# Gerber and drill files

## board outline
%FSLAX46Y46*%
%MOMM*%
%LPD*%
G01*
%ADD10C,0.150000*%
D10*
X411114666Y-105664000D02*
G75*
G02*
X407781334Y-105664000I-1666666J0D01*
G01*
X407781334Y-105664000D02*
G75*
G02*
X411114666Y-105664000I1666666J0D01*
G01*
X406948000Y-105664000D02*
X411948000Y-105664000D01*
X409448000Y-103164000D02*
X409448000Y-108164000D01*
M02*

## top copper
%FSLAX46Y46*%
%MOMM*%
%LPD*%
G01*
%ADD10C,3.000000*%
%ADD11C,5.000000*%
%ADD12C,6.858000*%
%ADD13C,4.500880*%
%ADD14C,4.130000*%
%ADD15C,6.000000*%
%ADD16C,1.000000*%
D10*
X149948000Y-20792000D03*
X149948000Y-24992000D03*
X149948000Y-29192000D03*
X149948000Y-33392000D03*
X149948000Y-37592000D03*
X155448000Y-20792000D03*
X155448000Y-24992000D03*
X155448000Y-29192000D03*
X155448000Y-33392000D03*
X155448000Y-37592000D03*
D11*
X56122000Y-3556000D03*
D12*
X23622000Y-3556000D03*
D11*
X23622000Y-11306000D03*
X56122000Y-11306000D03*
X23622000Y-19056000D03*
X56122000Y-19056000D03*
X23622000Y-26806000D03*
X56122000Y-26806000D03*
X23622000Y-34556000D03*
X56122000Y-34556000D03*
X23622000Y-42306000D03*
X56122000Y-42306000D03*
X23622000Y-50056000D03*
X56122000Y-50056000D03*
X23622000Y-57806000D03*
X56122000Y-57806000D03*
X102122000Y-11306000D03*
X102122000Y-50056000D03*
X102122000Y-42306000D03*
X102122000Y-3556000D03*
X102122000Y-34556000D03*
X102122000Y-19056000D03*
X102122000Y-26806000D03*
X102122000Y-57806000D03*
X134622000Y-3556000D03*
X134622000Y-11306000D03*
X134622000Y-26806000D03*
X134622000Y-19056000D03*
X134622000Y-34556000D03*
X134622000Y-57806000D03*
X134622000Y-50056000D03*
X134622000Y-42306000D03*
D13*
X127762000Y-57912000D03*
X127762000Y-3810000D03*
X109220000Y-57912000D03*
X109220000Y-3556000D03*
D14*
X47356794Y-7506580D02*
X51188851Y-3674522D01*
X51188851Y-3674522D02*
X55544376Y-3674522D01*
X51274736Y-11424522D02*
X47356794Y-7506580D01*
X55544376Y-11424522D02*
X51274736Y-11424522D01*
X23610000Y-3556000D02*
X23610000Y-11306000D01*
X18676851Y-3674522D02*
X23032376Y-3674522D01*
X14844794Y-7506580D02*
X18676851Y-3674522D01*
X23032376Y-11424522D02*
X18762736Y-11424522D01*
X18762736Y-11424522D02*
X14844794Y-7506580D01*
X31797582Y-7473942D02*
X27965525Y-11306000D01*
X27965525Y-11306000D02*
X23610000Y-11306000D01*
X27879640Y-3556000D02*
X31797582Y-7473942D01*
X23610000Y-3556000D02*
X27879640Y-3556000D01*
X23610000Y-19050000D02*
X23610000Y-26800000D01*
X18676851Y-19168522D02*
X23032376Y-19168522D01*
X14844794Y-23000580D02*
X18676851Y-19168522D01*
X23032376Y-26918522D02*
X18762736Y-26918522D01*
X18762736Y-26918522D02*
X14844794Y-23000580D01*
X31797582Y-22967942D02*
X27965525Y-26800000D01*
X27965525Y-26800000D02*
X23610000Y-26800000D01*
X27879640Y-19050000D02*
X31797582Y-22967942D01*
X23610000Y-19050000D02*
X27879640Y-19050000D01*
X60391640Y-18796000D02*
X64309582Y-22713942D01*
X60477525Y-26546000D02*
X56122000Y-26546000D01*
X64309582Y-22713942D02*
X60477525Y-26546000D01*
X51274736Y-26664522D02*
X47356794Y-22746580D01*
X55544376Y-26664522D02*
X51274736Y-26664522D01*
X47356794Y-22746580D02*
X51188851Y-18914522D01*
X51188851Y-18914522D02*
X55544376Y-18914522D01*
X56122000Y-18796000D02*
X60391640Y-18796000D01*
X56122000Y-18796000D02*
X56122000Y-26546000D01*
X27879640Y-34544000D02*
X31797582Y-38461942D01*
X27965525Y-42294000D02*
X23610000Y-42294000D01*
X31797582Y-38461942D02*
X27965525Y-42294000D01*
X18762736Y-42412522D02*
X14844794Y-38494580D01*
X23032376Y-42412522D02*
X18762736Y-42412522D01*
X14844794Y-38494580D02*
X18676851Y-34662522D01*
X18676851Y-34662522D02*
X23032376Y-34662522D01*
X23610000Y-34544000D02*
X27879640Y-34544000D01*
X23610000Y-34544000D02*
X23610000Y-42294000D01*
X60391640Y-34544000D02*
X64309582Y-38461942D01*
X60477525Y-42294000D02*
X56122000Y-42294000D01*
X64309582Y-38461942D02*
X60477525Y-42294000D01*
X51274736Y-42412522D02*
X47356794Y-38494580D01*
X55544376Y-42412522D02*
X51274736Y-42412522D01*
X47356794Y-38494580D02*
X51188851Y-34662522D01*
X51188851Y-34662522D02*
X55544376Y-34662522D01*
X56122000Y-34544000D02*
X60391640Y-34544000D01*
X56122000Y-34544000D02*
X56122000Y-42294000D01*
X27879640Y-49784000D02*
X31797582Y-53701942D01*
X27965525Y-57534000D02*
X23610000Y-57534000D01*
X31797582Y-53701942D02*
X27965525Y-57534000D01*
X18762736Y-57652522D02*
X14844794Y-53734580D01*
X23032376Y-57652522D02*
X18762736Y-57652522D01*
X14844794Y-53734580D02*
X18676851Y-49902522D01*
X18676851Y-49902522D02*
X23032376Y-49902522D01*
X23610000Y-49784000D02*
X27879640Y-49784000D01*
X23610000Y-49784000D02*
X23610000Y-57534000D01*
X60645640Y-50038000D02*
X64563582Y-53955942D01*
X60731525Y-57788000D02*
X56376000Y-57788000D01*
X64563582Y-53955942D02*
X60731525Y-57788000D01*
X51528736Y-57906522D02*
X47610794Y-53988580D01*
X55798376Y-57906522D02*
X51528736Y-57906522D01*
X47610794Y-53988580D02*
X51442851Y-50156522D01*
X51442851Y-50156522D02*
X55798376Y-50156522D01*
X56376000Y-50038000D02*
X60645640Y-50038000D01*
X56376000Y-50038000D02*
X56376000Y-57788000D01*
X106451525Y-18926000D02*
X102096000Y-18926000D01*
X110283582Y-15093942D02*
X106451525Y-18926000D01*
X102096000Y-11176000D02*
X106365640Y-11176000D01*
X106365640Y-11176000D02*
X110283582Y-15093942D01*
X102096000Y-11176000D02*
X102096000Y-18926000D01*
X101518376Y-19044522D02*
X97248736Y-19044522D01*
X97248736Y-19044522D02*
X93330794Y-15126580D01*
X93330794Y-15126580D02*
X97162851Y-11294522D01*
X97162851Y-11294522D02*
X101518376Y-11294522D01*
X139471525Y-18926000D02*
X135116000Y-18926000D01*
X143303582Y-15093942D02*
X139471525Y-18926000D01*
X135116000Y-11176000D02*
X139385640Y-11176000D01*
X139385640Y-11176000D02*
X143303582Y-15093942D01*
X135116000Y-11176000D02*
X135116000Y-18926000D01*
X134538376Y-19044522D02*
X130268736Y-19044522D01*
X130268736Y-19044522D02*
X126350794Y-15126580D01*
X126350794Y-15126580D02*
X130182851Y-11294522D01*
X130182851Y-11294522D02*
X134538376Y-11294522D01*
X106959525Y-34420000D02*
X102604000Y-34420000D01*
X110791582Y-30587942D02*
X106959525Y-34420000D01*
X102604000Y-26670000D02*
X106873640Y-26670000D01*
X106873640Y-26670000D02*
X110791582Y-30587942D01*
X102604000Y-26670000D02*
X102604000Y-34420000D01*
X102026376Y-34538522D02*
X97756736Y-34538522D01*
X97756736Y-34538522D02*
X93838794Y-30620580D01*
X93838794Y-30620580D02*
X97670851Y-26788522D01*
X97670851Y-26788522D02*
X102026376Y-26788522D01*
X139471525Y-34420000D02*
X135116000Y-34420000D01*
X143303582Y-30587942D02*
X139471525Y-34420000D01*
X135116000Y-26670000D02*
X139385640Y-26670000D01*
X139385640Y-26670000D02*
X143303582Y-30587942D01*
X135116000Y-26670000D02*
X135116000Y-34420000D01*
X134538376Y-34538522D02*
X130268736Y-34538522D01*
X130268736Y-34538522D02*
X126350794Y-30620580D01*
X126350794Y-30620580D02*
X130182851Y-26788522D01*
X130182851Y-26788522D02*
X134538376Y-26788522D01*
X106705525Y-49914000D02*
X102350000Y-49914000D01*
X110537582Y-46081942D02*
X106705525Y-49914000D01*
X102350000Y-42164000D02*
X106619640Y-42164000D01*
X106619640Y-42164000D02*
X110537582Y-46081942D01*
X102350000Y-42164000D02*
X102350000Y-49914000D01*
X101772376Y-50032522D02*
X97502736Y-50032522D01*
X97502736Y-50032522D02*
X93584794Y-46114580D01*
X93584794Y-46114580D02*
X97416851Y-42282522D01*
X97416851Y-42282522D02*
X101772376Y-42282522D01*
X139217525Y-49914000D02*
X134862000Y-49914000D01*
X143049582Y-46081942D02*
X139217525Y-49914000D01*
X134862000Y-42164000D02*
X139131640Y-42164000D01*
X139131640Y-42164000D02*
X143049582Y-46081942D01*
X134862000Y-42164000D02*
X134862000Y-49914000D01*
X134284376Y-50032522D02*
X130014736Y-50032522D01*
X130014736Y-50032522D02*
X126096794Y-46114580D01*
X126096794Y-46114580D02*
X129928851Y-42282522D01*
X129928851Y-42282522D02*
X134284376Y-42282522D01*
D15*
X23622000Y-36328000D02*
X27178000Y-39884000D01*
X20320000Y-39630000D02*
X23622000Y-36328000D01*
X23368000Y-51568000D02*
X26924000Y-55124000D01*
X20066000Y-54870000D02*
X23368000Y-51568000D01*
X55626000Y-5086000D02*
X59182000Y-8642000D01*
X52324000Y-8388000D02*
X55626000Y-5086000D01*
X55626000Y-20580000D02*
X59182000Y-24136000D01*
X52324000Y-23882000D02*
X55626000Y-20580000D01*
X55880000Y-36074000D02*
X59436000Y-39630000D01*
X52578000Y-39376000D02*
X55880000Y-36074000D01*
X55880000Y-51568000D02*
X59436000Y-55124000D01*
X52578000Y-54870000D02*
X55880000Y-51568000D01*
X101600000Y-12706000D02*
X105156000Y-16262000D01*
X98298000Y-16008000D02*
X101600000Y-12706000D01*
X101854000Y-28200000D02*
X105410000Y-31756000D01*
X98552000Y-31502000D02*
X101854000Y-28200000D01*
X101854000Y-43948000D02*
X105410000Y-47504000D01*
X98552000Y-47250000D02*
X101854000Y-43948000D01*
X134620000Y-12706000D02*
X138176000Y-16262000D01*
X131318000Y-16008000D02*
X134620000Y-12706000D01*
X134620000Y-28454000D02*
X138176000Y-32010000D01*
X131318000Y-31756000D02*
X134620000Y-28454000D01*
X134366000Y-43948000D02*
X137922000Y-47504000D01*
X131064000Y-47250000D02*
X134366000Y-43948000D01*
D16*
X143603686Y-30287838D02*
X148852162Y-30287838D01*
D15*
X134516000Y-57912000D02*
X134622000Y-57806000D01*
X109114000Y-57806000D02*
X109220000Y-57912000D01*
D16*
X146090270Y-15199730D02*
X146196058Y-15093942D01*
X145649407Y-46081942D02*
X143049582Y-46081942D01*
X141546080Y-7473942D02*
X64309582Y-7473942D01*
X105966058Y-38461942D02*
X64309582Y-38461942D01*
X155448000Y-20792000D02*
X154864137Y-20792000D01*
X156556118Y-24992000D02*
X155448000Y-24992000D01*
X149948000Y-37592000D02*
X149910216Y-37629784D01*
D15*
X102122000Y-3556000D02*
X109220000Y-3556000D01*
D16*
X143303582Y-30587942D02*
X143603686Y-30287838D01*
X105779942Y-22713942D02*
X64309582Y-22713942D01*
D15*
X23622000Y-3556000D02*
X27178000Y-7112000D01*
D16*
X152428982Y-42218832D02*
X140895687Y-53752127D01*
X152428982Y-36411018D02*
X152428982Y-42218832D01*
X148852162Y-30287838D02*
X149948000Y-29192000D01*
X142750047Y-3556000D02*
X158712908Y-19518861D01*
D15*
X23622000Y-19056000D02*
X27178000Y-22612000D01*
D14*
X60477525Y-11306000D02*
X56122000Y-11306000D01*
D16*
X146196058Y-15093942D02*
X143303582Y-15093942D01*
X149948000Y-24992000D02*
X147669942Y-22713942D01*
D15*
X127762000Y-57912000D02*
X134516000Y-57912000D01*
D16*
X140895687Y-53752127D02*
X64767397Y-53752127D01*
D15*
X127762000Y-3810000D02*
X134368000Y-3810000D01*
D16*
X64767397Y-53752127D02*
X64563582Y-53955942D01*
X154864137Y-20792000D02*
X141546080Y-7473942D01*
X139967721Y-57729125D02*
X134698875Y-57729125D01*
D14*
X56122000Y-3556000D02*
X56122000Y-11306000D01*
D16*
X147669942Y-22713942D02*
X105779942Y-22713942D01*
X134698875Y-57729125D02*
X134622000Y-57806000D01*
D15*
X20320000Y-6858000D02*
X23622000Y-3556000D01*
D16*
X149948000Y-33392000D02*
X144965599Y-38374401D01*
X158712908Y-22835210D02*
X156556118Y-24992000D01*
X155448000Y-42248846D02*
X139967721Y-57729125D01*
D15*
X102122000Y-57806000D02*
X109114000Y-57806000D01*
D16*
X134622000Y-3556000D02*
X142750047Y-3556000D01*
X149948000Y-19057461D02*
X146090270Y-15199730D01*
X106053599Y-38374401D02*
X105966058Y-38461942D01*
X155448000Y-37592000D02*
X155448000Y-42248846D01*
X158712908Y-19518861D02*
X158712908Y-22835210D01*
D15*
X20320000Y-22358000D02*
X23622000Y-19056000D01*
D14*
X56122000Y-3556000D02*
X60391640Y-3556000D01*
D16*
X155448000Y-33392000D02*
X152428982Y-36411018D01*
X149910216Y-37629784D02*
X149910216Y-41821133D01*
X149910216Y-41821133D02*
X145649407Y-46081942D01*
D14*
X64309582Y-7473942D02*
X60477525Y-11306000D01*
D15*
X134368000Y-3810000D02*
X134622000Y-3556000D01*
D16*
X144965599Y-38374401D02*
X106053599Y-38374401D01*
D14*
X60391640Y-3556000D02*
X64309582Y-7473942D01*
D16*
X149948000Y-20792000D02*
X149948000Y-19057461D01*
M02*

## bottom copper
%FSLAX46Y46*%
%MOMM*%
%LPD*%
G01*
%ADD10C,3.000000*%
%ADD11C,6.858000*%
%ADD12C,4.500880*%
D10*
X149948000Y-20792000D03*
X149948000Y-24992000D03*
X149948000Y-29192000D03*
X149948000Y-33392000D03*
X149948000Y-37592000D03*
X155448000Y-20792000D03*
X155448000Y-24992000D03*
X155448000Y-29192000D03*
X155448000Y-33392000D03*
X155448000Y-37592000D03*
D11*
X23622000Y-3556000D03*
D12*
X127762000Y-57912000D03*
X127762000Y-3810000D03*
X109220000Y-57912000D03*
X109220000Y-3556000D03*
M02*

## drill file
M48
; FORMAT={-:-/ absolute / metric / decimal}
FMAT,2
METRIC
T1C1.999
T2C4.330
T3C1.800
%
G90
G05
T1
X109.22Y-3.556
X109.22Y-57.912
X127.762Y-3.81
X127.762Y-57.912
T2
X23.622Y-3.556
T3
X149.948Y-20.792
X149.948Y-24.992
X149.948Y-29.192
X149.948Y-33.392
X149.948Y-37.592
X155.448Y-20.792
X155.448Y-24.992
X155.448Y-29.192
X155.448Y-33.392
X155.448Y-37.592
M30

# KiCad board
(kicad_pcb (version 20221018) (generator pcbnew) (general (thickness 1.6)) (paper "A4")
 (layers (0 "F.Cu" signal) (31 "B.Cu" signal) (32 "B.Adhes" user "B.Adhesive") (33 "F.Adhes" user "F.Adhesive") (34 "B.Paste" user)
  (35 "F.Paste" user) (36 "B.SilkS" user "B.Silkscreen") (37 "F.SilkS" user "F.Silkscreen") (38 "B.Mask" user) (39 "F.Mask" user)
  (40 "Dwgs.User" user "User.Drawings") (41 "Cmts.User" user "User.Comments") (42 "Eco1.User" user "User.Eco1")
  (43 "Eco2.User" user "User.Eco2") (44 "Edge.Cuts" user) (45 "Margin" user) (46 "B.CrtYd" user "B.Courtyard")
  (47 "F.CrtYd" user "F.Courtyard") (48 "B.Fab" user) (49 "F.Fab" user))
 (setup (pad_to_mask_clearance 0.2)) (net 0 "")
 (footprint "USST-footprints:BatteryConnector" (layer "F.Cu") (at 149.948 37.592)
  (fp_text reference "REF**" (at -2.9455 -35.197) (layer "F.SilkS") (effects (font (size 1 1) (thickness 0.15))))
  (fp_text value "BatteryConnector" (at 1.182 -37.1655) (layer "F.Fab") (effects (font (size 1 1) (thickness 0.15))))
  (pad "" np_thru_hole circle (at 0 -16.8) (size 3 3) (drill 1.8) (layers "*.Cu"))
  (pad "" np_thru_hole circle (at 0 -12.6) (size 3 3) (drill 1.8) (layers "*.Cu"))
  (pad "" np_thru_hole circle (at 0 -8.4) (size 3 3) (drill 1.8) (layers "*.Cu"))
  (pad "" np_thru_hole circle (at 0 -4.2) (size 3 3) (drill 1.8) (layers "*.Cu"))
  (pad "" np_thru_hole circle (at 0 0) (size 3 3) (drill 1.8) (layers "*.Cu"))
  (pad "" np_thru_hole circle (at 5.5 -16.8) (size 3 3) (drill 1.8) (layers "*.Cu"))
  (pad "" np_thru_hole circle (at 5.5 -12.6) (size 3 3) (drill 1.8) (layers "*.Cu"))
  (pad "" np_thru_hole circle (at 5.5 -8.4) (size 3 3) (drill 1.8) (layers "*.Cu"))
  (pad "" np_thru_hole circle (at 5.5 -4.2) (size 3 3) (drill 1.8) (layers "*.Cu"))
  (pad "" np_thru_hole circle (at 5.5 0) (size 3 3) (drill 1.8) (layers "*.Cu")))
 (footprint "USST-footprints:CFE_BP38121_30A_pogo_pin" (layer "F.Cu") (at 96 14.986)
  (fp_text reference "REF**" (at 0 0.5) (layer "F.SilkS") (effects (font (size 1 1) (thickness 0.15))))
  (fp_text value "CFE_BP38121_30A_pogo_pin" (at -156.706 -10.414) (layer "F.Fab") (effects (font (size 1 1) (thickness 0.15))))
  (pad "1" smd circle (at -39.878 -11.43) (size 5 5) (layers "F.Cu" "F.Paste" "F.Mask")))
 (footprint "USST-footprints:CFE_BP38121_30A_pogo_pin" (layer "F.Cu") (at 63.5 14.986)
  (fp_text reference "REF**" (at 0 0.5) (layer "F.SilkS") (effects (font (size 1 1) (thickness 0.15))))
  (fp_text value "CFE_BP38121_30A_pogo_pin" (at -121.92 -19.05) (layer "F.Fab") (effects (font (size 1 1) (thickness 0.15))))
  (pad "1" thru_hole circle (at -39.878 -11.43) (size 6.858 6.858) (drill 4.33) (layers "*.Cu" "*.Mask")))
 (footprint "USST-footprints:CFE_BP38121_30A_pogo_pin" (layer "F.Cu") (at 63.5 22.736)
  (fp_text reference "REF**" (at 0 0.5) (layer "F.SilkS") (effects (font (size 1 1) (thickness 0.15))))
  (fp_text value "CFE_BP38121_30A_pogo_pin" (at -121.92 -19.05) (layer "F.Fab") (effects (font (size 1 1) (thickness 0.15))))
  (pad "2" smd circle (at -39.878 -11.43) (size 5 5) (layers "F.Cu" "F.Paste" "F.Mask")))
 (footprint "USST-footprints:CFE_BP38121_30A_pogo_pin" (layer "F.Cu") (at 96 22.736)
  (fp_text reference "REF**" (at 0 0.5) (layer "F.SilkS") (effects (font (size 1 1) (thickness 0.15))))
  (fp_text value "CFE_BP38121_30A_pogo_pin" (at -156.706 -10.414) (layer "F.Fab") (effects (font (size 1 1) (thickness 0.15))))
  (pad "2" smd circle (at -39.878 -11.43) (size 5 5) (layers "F.Cu" "F.Paste" "F.Mask")))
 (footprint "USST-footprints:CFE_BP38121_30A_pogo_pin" (layer "F.Cu") (at 63.5 30.486)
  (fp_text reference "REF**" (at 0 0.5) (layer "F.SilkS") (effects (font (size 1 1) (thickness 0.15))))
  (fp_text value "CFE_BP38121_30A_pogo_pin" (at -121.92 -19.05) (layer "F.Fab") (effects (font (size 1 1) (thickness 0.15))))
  (pad "3" smd circle (at -39.878 -11.43) (size 5 5) (layers "F.Cu" "F.Paste" "F.Mask")))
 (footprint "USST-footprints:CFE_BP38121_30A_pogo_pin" (layer "F.Cu") (at 96 30.486)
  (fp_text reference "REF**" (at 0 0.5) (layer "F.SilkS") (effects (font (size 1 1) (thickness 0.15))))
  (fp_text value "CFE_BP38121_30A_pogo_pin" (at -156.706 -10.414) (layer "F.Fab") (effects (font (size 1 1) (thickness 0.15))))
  (pad "3" smd circle (at -39.878 -11.43) (size 5 5) (layers "F.Cu" "F.Paste" "F.Mask")))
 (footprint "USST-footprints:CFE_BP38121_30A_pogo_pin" (layer "F.Cu") (at 63.5 38.236)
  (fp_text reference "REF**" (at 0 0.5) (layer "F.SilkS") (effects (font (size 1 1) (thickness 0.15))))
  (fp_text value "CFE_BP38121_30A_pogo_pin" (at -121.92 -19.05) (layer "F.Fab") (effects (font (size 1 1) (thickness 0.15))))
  (pad "4" smd circle (at -39.878 -11.43) (size 5 5) (layers "F.Cu" "F.Paste" "F.Mask")))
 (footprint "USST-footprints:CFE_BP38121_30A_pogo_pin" (layer "F.Cu") (at 96 38.236)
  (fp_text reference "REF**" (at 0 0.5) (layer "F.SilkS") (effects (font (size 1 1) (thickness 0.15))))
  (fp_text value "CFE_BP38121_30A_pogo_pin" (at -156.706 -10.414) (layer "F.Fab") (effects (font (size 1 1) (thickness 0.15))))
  (pad "4" smd circle (at -39.878 -11.43) (size 5 5) (layers "F.Cu" "F.Paste" "F.Mask")))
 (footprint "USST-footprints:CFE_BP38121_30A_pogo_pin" (layer "F.Cu") (at 63.5 45.986)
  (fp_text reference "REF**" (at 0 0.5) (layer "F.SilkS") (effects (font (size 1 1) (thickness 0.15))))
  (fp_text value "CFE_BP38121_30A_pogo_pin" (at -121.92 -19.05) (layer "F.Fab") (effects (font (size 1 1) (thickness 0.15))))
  (pad "5" smd circle (at -39.878 -11.43) (size 5 5) (layers "F.Cu" "F.Paste" "F.Mask")))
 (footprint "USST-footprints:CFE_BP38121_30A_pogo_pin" (layer "F.Cu") (at 96 45.986)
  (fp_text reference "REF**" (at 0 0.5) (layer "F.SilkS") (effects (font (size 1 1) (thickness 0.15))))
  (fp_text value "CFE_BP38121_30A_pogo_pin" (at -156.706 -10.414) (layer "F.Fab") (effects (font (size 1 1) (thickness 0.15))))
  (pad "5" smd circle (at -39.878 -11.43) (size 5 5) (layers "F.Cu" "F.Paste" "F.Mask")))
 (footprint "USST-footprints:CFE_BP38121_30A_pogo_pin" (layer "F.Cu") (at 63.5 53.736)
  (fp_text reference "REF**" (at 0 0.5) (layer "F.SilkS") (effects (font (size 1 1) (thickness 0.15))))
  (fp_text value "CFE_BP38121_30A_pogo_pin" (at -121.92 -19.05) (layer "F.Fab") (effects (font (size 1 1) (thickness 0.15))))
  (pad "6" smd circle (at -39.878 -11.43) (size 5 5) (layers "F.Cu" "F.Paste" "F.Mask")))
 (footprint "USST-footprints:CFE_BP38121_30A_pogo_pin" (layer "F.Cu") (at 96 53.736)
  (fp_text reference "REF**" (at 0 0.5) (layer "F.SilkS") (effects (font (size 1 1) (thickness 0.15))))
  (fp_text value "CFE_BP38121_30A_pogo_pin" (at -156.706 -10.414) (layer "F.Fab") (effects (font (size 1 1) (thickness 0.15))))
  (pad "6" smd circle (at -39.878 -11.43) (size 5 5) (layers "F.Cu" "F.Paste" "F.Mask")))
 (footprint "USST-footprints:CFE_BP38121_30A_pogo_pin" (layer "F.Cu") (at 63.5 61.486)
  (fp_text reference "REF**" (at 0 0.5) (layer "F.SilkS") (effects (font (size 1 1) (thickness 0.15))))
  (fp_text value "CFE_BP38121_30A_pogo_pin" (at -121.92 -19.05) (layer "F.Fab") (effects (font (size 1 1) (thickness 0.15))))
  (pad "7" smd circle (at -39.878 -11.43) (size 5 5) (layers "F.Cu" "F.Paste" "F.Mask")))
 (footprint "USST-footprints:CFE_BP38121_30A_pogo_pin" (layer "F.Cu") (at 96 61.486)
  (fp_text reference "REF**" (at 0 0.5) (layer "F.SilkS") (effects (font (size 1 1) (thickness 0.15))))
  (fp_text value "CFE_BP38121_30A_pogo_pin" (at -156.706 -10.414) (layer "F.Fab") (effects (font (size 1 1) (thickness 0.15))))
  (pad "7" smd circle (at -39.878 -11.43) (size 5 5) (layers "F.Cu" "F.Paste" "F.Mask")))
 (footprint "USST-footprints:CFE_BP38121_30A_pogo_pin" (layer "F.Cu") (at 63.5 69.236)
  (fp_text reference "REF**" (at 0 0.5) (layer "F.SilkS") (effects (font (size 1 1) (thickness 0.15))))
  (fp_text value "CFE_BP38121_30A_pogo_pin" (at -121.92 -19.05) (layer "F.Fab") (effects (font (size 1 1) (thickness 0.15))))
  (pad "8" smd circle (at -39.878 -11.43) (size 5 5) (layers "F.Cu" "F.Paste" "F.Mask")))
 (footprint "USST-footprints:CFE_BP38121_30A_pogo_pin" (layer "F.Cu") (at 96 69.236)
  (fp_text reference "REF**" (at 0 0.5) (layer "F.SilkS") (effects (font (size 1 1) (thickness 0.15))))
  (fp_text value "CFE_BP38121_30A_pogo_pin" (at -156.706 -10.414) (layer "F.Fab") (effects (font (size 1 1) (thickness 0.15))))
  (pad "8" smd circle (at -39.878 -11.43) (size 5 5) (layers "F.Cu" "F.Paste" "F.Mask")))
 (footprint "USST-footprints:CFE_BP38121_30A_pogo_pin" (layer "F.Cu") (at 142 22.736)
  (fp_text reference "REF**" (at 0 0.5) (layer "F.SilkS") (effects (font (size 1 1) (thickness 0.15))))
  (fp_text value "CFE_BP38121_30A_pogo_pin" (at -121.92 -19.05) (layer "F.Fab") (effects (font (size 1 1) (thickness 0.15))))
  (pad "2" smd circle (at -39.878 -11.43) (size 5 5) (layers "F.Cu" "F.Paste" "F.Mask")))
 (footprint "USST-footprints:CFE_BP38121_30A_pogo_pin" (layer "F.Cu") (at 142 61.486)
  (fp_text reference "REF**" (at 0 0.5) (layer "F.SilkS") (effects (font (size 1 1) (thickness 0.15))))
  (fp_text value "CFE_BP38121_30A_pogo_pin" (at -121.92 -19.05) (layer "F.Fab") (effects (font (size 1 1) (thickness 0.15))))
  (pad "7" smd circle (at -39.878 -11.43) (size 5 5) (layers "F.Cu" "F.Paste" "F.Mask")))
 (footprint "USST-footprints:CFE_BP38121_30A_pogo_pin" (layer "F.Cu") (at 142 53.736)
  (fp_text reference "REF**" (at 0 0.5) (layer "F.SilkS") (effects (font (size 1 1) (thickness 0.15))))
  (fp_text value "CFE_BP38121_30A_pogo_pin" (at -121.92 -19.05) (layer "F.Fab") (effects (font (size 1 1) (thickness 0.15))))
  (pad "6" smd circle (at -39.878 -11.43) (size 5 5) (layers "F.Cu" "F.Paste" "F.Mask")))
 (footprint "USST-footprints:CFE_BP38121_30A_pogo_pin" (layer "F.Cu") (at 142 14.986)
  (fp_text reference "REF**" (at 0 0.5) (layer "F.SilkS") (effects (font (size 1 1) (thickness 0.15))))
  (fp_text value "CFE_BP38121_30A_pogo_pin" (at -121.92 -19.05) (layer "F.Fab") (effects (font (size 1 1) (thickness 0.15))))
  (pad "1" smd circle (at -39.878 -11.43) (size 5 5) (layers "F.Cu" "F.Paste" "F.Mask")))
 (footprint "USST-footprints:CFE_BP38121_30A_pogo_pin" (layer "F.Cu") (at 142 45.986)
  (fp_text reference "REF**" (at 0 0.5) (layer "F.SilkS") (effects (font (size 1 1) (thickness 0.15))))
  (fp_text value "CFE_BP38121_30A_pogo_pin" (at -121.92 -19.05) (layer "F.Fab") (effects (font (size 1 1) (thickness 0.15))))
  (pad "5" smd circle (at -39.878 -11.43) (size 5 5) (layers "F.Cu" "F.Paste" "F.Mask")))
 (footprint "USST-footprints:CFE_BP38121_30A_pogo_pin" (layer "F.Cu") (at 142 30.486)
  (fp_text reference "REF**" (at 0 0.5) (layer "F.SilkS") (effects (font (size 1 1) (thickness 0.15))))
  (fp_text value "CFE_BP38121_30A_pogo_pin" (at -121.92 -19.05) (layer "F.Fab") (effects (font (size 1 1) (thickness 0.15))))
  (pad "3" smd circle (at -39.878 -11.43) (size 5 5) (layers "F.Cu" "F.Paste" "F.Mask")))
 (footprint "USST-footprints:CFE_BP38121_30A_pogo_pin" (layer "F.Cu") (at 142 38.236)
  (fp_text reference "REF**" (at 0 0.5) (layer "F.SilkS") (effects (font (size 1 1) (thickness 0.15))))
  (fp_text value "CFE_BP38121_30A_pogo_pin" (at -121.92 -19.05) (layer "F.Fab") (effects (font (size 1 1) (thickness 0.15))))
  (pad "4" smd circle (at -39.878 -11.43) (size 5 5) (layers "F.Cu" "F.Paste" "F.Mask")))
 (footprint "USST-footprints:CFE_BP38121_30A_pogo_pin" (layer "F.Cu") (at 142 69.236)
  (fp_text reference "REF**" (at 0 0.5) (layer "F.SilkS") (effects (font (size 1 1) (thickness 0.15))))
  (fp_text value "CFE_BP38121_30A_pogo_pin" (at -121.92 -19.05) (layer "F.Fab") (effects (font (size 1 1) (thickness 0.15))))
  (pad "8" smd circle (at -39.878 -11.43) (size 5 5) (layers "F.Cu" "F.Paste" "F.Mask")))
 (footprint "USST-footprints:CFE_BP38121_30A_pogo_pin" (layer "F.Cu") (at 174.5 14.986)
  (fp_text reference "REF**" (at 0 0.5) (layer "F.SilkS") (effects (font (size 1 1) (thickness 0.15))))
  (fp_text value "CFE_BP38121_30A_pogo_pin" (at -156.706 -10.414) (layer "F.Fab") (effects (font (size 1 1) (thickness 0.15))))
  (pad "1" smd circle (at -39.878 -11.43) (size 5 5) (layers "F.Cu" "F.Paste" "F.Mask")))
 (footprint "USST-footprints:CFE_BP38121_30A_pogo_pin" (layer "F.Cu") (at 174.5 22.736)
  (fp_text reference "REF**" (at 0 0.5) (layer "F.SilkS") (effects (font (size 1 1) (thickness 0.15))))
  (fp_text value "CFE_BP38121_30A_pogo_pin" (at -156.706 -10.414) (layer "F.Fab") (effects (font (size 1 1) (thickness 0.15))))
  (pad "2" smd circle (at -39.878 -11.43) (size 5 5) (layers "F.Cu" "F.Paste" "F.Mask")))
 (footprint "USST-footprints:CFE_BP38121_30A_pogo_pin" (layer "F.Cu") (at 174.5 38.236)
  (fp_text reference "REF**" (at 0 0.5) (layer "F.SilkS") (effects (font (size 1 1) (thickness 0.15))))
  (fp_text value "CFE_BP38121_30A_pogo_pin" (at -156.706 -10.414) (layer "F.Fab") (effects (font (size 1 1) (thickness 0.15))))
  (pad "4" smd circle (at -39.878 -11.43) (size 5 5) (layers "F.Cu" "F.Paste" "F.Mask")))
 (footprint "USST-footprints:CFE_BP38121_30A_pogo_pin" (layer "F.Cu") (at 174.5 30.486)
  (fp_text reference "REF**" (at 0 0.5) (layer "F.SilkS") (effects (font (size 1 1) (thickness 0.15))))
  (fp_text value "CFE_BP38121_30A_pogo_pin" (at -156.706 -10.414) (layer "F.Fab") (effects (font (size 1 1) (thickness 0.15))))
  (pad "3" smd circle (at -39.878 -11.43) (size 5 5) (layers "F.Cu" "F.Paste" "F.Mask")))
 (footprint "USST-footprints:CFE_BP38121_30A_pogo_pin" (layer "F.Cu") (at 174.5 45.986)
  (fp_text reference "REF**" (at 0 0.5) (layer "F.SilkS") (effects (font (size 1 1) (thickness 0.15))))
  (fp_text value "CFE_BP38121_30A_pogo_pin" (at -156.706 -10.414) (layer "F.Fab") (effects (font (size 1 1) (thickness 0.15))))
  (pad "5" smd circle (at -39.878 -11.43) (size 5 5) (layers "F.Cu" "F.Paste" "F.Mask")))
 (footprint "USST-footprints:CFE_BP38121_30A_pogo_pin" (layer "F.Cu") (at 174.5 69.236)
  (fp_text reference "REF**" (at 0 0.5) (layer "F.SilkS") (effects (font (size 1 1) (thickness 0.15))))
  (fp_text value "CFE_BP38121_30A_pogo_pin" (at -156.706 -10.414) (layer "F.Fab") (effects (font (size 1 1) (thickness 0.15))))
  (pad "8" smd circle (at -39.878 -11.43) (size 5 5) (layers "F.Cu" "F.Paste" "F.Mask")))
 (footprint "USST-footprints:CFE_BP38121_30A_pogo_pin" (layer "F.Cu") (at 174.5 61.486)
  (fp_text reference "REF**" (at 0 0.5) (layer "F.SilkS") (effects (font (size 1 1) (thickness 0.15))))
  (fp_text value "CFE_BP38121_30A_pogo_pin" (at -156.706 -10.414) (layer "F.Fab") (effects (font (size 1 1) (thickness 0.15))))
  (pad "7" smd circle (at -39.878 -11.43) (size 5 5) (layers "F.Cu" "F.Paste" "F.Mask")))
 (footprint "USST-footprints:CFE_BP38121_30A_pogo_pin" (layer "F.Cu") (at 174.5 53.736)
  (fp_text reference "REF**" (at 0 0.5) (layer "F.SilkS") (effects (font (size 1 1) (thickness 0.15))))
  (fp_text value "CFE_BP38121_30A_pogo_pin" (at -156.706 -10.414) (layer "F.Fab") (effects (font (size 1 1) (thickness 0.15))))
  (pad "6" smd circle (at -39.878 -11.43) (size 5 5) (layers "F.Cu" "F.Paste" "F.Mask")))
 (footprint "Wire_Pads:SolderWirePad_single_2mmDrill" (layer "F.Cu") (at 127.762 57.912)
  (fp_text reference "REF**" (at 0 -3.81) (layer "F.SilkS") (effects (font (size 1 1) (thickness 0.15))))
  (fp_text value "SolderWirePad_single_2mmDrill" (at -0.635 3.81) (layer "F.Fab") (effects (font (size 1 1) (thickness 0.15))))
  (pad "1" thru_hole circle (at 0 0) (size 4.50088 4.50088) (drill 1.99898) (layers "*.Cu" "*.Mask")))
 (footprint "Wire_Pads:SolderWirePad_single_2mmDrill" (layer "F.Cu") (at 127.762 3.81)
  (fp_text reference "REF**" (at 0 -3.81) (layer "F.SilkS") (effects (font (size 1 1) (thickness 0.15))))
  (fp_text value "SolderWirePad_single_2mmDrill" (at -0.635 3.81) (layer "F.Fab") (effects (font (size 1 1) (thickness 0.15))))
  (pad "1" thru_hole circle (at 0 0) (size 4.50088 4.50088) (drill 1.99898) (layers "*.Cu" "*.Mask")))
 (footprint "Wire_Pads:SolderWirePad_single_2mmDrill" (layer "F.Cu") (at 109.22 57.912)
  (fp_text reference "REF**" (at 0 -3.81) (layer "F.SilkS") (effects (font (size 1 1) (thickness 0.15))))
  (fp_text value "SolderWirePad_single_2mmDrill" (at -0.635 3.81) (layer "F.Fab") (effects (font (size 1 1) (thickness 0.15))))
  (pad "1" thru_hole circle (at 0 0) (size 4.50088 4.50088) (drill 1.99898) (layers "*.Cu" "*.Mask")))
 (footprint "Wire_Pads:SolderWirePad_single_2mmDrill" (layer "F.Cu") (at 109.22 3.556)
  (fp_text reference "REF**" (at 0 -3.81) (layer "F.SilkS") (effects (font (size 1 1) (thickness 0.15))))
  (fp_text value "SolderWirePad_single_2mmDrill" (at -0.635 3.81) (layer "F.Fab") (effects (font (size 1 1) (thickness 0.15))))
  (pad "1" thru_hole circle (at 0 0) (size 4.50088 4.50088) (drill 1.99898) (layers "*.Cu" "*.Mask")))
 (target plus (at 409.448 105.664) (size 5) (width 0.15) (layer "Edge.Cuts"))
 (segment (start 47.356794 7.50658) (end 51.188851 3.674522) (width 4.13) (layer "F.Cu") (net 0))
 (segment (start 51.188851 3.674522) (end 55.544376 3.674522) (width 4.13) (layer "F.Cu") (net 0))
 (segment (start 51.274736 11.424522) (end 47.356794 7.50658) (width 4.13) (layer "F.Cu") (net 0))
 (segment (start 55.544376 11.424522) (end 51.274736 11.424522) (width 4.13) (layer "F.Cu") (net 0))
 (segment (start 23.61 3.556) (end 23.61 11.306) (width 4.13) (layer "F.Cu") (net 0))
 (segment (start 18.676851 3.674522) (end 23.032376 3.674522) (width 4.13) (layer "F.Cu") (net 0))
 (segment (start 14.844794 7.50658) (end 18.676851 3.674522) (width 4.13) (layer "F.Cu") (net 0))
 (segment (start 23.032376 11.424522) (end 18.762736 11.424522) (width 4.13) (layer "F.Cu") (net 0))
 (segment (start 18.762736 11.424522) (end 14.844794 7.50658) (width 4.13) (layer "F.Cu") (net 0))
 (segment (start 31.797582 7.473942) (end 27.965525 11.306) (width 4.13) (layer "F.Cu") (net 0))
 (segment (start 27.965525 11.306) (end 23.61 11.306) (width 4.13) (layer "F.Cu") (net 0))
 (segment (start 27.87964 3.556) (end 31.797582 7.473942) (width 4.13) (layer "F.Cu") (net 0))
 (segment (start 23.61 3.556) (end 27.87964 3.556) (width 4.13) (layer "F.Cu") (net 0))
 (segment (start 23.61 19.05) (end 23.61 26.8) (width 4.13) (layer "F.Cu") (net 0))
 (segment (start 18.676851 19.168522) (end 23.032376 19.168522) (width 4.13) (layer "F.Cu") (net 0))
 (segment (start 14.844794 23.00058) (end 18.676851 19.168522) (width 4.13) (layer "F.Cu") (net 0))
 (segment (start 23.032376 26.918522) (end 18.762736 26.918522) (width 4.13) (layer "F.Cu") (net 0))
 (segment (start 18.762736 26.918522) (end 14.844794 23.00058) (width 4.13) (layer "F.Cu") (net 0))
 (segment (start 31.797582 22.967942) (end 27.965525 26.8) (width 4.13) (layer "F.Cu") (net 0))
 (segment (start 27.965525 26.8) (end 23.61 26.8) (width 4.13) (layer "F.Cu") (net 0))
 (segment (start 27.87964 19.05) (end 31.797582 22.967942) (width 4.13) (layer "F.Cu") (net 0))
 (segment (start 23.61 19.05) (end 27.87964 19.05) (width 4.13) (layer "F.Cu") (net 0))
 (segment (start 60.39164 18.796) (end 64.309582 22.713942) (width 4.13) (layer "F.Cu") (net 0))
 (segment (start 60.477525 26.546) (end 56.122 26.546) (width 4.13) (layer "F.Cu") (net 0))
 (segment (start 64.309582 22.713942) (end 60.477525 26.546) (width 4.13) (layer "F.Cu") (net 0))
 (segment (start 51.274736 26.664522) (end 47.356794 22.74658) (width 4.13) (layer "F.Cu") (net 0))
 (segment (start 55.544376 26.664522) (end 51.274736 26.664522) (width 4.13) (layer "F.Cu") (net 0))
 (segment (start 47.356794 22.74658) (end 51.188851 18.914522) (width 4.13) (layer "F.Cu") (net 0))
 (segment (start 51.188851 18.914522) (end 55.544376 18.914522) (width 4.13) (layer "F.Cu") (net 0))
 (segment (start 56.122 18.796) (end 60.39164 18.796) (width 4.13) (layer "F.Cu") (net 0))
 (segment (start 56.122 18.796) (end 56.122 26.546) (width 4.13) (layer "F.Cu") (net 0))
 (segment (start 27.87964 34.544) (end 31.797582 38.461942) (width 4.13) (layer "F.Cu") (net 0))
 (segment (start 27.965525 42.294) (end 23.61 42.294) (width 4.13) (layer "F.Cu") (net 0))
 (segment (start 31.797582 38.461942) (end 27.965525 42.294) (width 4.13) (layer "F.Cu") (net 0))
 (segment (start 18.762736 42.412522) (end 14.844794 38.49458) (width 4.13) (layer "F.Cu") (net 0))
 (segment (start 23.032376 42.412522) (end 18.762736 42.412522) (width 4.13) (layer "F.Cu") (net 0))
 (segment (start 14.844794 38.49458) (end 18.676851 34.662522) (width 4.13) (layer "F.Cu") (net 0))
 (segment (start 18.676851 34.662522) (end 23.032376 34.662522) (width 4.13) (layer "F.Cu") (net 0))
 (segment (start 23.61 34.544) (end 27.87964 34.544) (width 4.13) (layer "F.Cu") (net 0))
 (segment (start 23.61 34.544) (end 23.61 42.294) (width 4.13) (layer "F.Cu") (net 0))
 (segment (start 60.39164 34.544) (end 64.309582 38.461942) (width 4.13) (layer "F.Cu") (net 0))
 (segment (start 60.477525 42.294) (end 56.122 42.294) (width 4.13) (layer "F.Cu") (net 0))
 (segment (start 64.309582 38.461942) (end 60.477525 42.294) (width 4.13) (layer "F.Cu") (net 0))
 (segment (start 51.274736 42.412522) (end 47.356794 38.49458) (width 4.13) (layer "F.Cu") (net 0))
 (segment (start 55.544376 42.412522) (end 51.274736 42.412522) (width 4.13) (layer "F.Cu") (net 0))
 (segment (start 47.356794 38.49458) (end 51.188851 34.662522) (width 4.13) (layer "F.Cu") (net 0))
 (segment (start 51.188851 34.662522) (end 55.544376 34.662522) (width 4.13) (layer "F.Cu") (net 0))
 (segment (start 56.122 34.544) (end 60.39164 34.544) (width 4.13) (layer "F.Cu") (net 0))
 (segment (start 56.122 34.544) (end 56.122 42.294) (width 4.13) (layer "F.Cu") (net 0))
 (segment (start 27.87964 49.784) (end 31.797582 53.701942) (width 4.13) (layer "F.Cu") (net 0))
 (segment (start 27.965525 57.534) (end 23.61 57.534) (width 4.13) (layer "F.Cu") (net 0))
 (segment (start 31.797582 53.701942) (end 27.965525 57.534) (width 4.13) (layer "F.Cu") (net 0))
 (segment (start 18.762736 57.652522) (end 14.844794 53.73458) (width 4.13) (layer "F.Cu") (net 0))
 (segment (start 23.032376 57.652522) (end 18.762736 57.652522) (width 4.13) (layer "F.Cu") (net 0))
 (segment (start 14.844794 53.73458) (end 18.676851 49.902522) (width 4.13) (layer "F.Cu") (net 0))
 (segment (start 18.676851 49.902522) (end 23.032376 49.902522) (width 4.13) (layer "F.Cu") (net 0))
 (segment (start 23.61 49.784) (end 27.87964 49.784) (width 4.13) (layer "F.Cu") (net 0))
 (segment (start 23.61 49.784) (end 23.61 57.534) (width 4.13) (layer "F.Cu") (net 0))
 (segment (start 60.64564 50.038) (end 64.563582 53.955942) (width 4.13) (layer "F.Cu") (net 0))
 (segment (start 60.731525 57.788) (end 56.376 57.788) (width 4.13) (layer "F.Cu") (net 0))
 (segment (start 64.563582 53.955942) (end 60.731525 57.788) (width 4.13) (layer "F.Cu") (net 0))
 (segment (start 51.528736 57.906522) (end 47.610794 53.98858) (width 4.13) (layer "F.Cu") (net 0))
 (segment (start 55.798376 57.906522) (end 51.528736 57.906522) (width 4.13) (layer "F.Cu") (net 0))
 (segment (start 47.610794 53.98858) (end 51.442851 50.156522) (width 4.13) (layer "F.Cu") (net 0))
 (segment (start 51.442851 50.156522) (end 55.798376 50.156522) (width 4.13) (layer "F.Cu") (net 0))
 (segment (start 56.376 50.038) (end 60.64564 50.038) (width 4.13) (layer "F.Cu") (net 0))
 (segment (start 56.376 50.038) (end 56.376 57.788) (width 4.13) (layer "F.Cu") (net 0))
 (segment (start 106.451525 18.926) (end 102.096 18.926) (width 4.13) (layer "F.Cu") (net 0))
 (segment (start 110.283582 15.093942) (end 106.451525 18.926) (width 4.13) (layer "F.Cu") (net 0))
 (segment (start 102.096 11.176) (end 106.36564 11.176) (width 4.13) (layer "F.Cu") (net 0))
 (segment (start 106.36564 11.176) (end 110.283582 15.093942) (width 4.13) (layer "F.Cu") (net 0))
 (segment (start 102.096 11.176) (end 102.096 18.926) (width 4.13) (layer "F.Cu") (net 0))
 (segment (start 101.518376 19.044522) (end 97.248736 19.044522) (width 4.13) (layer "F.Cu") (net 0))
 (segment (start 97.248736 19.044522) (end 93.330794 15.12658) (width 4.13) (layer "F.Cu") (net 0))
 (segment (start 93.330794 15.12658) (end 97.162851 11.294522) (width 4.13) (layer "F.Cu") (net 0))
 (segment (start 97.162851 11.294522) (end 101.518376 11.294522) (width 4.13) (layer "F.Cu") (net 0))
 (segment (start 139.471525 18.926) (end 135.116 18.926) (width 4.13) (layer "F.Cu") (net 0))
 (segment (start 143.303582 15.093942) (end 139.471525 18.926) (width 4.13) (layer "F.Cu") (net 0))
 (segment (start 135.116 11.176) (end 139.38564 11.176) (width 4.13) (layer "F.Cu") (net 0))
 (segment (start 139.38564 11.176) (end 143.303582 15.093942) (width 4.13) (layer "F.Cu") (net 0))
 (segment (start 135.116 11.176) (end 135.116 18.926) (width 4.13) (layer "F.Cu") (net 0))
 (segment (start 134.538376 19.044522) (end 130.268736 19.044522) (width 4.13) (layer "F.Cu") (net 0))
 (segment (start 130.268736 19.044522) (end 126.350794 15.12658) (width 4.13) (layer "F.Cu") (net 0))
 (segment (start 126.350794 15.12658) (end 130.182851 11.294522) (width 4.13) (layer "F.Cu") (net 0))
 (segment (start 130.182851 11.294522) (end 134.538376 11.294522) (width 4.13) (layer "F.Cu") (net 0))
 (segment (start 106.959525 34.42) (end 102.604 34.42) (width 4.13) (layer "F.Cu") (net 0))
 (segment (start 110.791582 30.587942) (end 106.959525 34.42) (width 4.13) (layer "F.Cu") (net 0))
 (segment (start 102.604 26.67) (end 106.87364 26.67) (width 4.13) (layer "F.Cu") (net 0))
 (segment (start 106.87364 26.67) (end 110.791582 30.587942) (width 4.13) (layer "F.Cu") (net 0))
 (segment (start 102.604 26.67) (end 102.604 34.42) (width 4.13) (layer "F.Cu") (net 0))
 (segment (start 102.026376 34.538522) (end 97.756736 34.538522) (width 4.13) (layer "F.Cu") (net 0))
 (segment (start 97.756736 34.538522) (end 93.838794 30.62058) (width 4.13) (layer "F.Cu") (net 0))
 (segment (start 93.838794 30.62058) (end 97.670851 26.788522) (width 4.13) (layer "F.Cu") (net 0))
 (segment (start 97.670851 26.788522) (end 102.026376 26.788522) (width 4.13) (layer "F.Cu") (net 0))
 (segment (start 139.471525 34.42) (end 135.116 34.42) (width 4.13) (layer "F.Cu") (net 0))
 (segment (start 143.303582 30.587942) (end 139.471525 34.42) (width 4.13) (layer "F.Cu") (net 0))
 (segment (start 135.116 26.67) (end 139.38564 26.67) (width 4.13) (layer "F.Cu") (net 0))
 (segment (start 139.38564 26.67) (end 143.303582 30.587942) (width 4.13) (layer "F.Cu") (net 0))
 (segment (start 135.116 26.67) (end 135.116 34.42) (width 4.13) (layer "F.Cu") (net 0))
 (segment (start 134.538376 34.538522) (end 130.268736 34.538522) (width 4.13) (layer "F.Cu") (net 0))
 (segment (start 130.268736 34.538522) (end 126.350794 30.62058) (width 4.13) (layer "F.Cu") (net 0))
 (segment (start 126.350794 30.62058) (end 130.182851 26.788522) (width 4.13) (layer "F.Cu") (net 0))
 (segment (start 130.182851 26.788522) (end 134.538376 26.788522) (width 4.13) (layer "F.Cu") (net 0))
 (segment (start 106.705525 49.914) (end 102.35 49.914) (width 4.13) (layer "F.Cu") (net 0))
 (segment (start 110.537582 46.081942) (end 106.705525 49.914) (width 4.13) (layer "F.Cu") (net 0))
 (segment (start 102.35 42.164) (end 106.61964 42.164) (width 4.13) (layer "F.Cu") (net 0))
 (segment (start 106.61964 42.164) (end 110.537582 46.081942) (width 4.13) (layer "F.Cu") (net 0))
 (segment (start 102.35 42.164) (end 102.35 49.914) (width 4.13) (layer "F.Cu") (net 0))
 (segment (start 101.772376 50.032522) (end 97.502736 50.032522) (width 4.13) (layer "F.Cu") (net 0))
 (segment (start 97.502736 50.032522) (end 93.584794 46.11458) (width 4.13) (layer "F.Cu") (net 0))
 (segment (start 93.584794 46.11458) (end 97.416851 42.282522) (width 4.13) (layer "F.Cu") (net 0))
 (segment (start 97.416851 42.282522) (end 101.772376 42.282522) (width 4.13) (layer "F.Cu") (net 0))
 (segment (start 139.217525 49.914) (end 134.862 49.914) (width 4.13) (layer "F.Cu") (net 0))
 (segment (start 143.049582 46.081942) (end 139.217525 49.914) (width 4.13) (layer "F.Cu") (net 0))
 (segment (start 134.862 42.164) (end 139.13164 42.164) (width 4.13) (layer "F.Cu") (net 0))
 (segment (start 139.13164 42.164) (end 143.049582 46.081942) (width 4.13) (layer "F.Cu") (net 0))
 (segment (start 134.862 42.164) (end 134.862 49.914) (width 4.13) (layer "F.Cu") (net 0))
 (segment (start 134.284376 50.032522) (end 130.014736 50.032522) (width 4.13) (layer "F.Cu") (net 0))
 (segment (start 130.014736 50.032522) (end 126.096794 46.11458) (width 4.13) (layer "F.Cu") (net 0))
 (segment (start 126.096794 46.11458) (end 129.928851 42.282522) (width 4.13) (layer "F.Cu") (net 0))
 (segment (start 129.928851 42.282522) (end 134.284376 42.282522) (width 4.13) (layer "F.Cu") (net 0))
 (segment (start 23.622 36.328) (end 27.178 39.884) (width 6) (layer "F.Cu") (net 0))
 (segment (start 20.32 39.63) (end 23.622 36.328) (width 6) (layer "F.Cu") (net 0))
 (segment (start 23.368 51.568) (end 26.924 55.124) (width 6) (layer "F.Cu") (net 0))
 (segment (start 20.066 54.87) (end 23.368 51.568) (width 6) (layer "F.Cu") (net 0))
 (segment (start 55.626 5.086) (end 59.182 8.642) (width 6) (layer "F.Cu") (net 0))
 (segment (start 52.324 8.388) (end 55.626 5.086) (width 6) (layer "F.Cu") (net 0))
 (segment (start 55.626 20.58) (end 59.182 24.136) (width 6) (layer "F.Cu") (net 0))
 (segment (start 52.324 23.882) (end 55.626 20.58) (width 6) (layer "F.Cu") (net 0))
 (segment (start 55.88 36.074) (end 59.436 39.63) (width 6) (layer "F.Cu") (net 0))
 (segment (start 52.578 39.376) (end 55.88 36.074) (width 6) (layer "F.Cu") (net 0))
 (segment (start 55.88 51.568) (end 59.436 55.124) (width 6) (layer "F.Cu") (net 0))
 (segment (start 52.578 54.87) (end 55.88 51.568) (width 6) (layer "F.Cu") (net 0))
 (segment (start 101.6 12.706) (end 105.156 16.262) (width 6) (layer "F.Cu") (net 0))
 (segment (start 98.298 16.008) (end 101.6 12.706) (width 6) (layer "F.Cu") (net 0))
 (segment (start 101.854 28.2) (end 105.41 31.756) (width 6) (layer "F.Cu") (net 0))
 (segment (start 98.552 31.502) (end 101.854 28.2) (width 6) (layer "F.Cu") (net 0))
 (segment (start 101.854 43.948) (end 105.41 47.504) (width 6) (layer "F.Cu") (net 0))
 (segment (start 98.552 47.25) (end 101.854 43.948) (width 6) (layer "F.Cu") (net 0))
 (segment (start 134.62 12.706) (end 138.176 16.262) (width 6) (layer "F.Cu") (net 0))
 (segment (start 131.318 16.008) (end 134.62 12.706) (width 6) (layer "F.Cu") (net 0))
 (segment (start 134.62 28.454) (end 138.176 32.01) (width 6) (layer "F.Cu") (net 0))
 (segment (start 131.318 31.756) (end 134.62 28.454) (width 6) (layer "F.Cu") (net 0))
 (segment (start 134.366 43.948) (end 137.922 47.504) (width 6) (layer "F.Cu") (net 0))
 (segment (start 131.064 47.25) (end 134.366 43.948) (width 6) (layer "F.Cu") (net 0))
 (segment (start 143.603686 30.287838) (end 148.852162 30.287838) (width 1) (layer "F.Cu") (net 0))
 (segment (start 134.516 57.912) (end 134.622 57.806) (width 6) (layer "F.Cu") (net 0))
 (segment (start 109.114 57.806) (end 109.22 57.912) (width 6) (layer "F.Cu") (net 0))
 (segment (start 146.09027 15.19973) (end 146.196058 15.093942) (width 1) (layer "F.Cu") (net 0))
 (segment (start 145.649407 46.081942) (end 143.049582 46.081942) (width 1) (layer "F.Cu") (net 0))
 (segment (start 141.54608 7.473942) (end 64.309582 7.473942) (width 1) (layer "F.Cu") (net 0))
 (segment (start 105.966058 38.461942) (end 64.309582 38.461942) (width 1) (layer "F.Cu") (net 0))
 (segment (start 155.448 20.792) (end 154.864137 20.792) (width 1) (layer "F.Cu") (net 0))
 (segment (start 156.556118 24.992) (end 155.448 24.992) (width 1) (layer "F.Cu") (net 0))
 (segment (start 149.948 37.592) (end 149.910216 37.629784) (width 1) (layer "F.Cu") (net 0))
 (segment (start 102.122 3.556) (end 109.22 3.556) (width 6) (layer "F.Cu") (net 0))
 (segment (start 143.303582 30.587942) (end 143.603686 30.287838) (width 1) (layer "F.Cu") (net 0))
 (segment (start 105.779942 22.713942) (end 64.309582 22.713942) (width 1) (layer "F.Cu") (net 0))
 (segment (start 23.622 3.556) (end 27.178 7.112) (width 6) (layer "F.Cu") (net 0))
 (segment (start 152.428982 42.218832) (end 140.895687 53.752127) (width 1) (layer "F.Cu") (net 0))
 (segment (start 152.428982 36.411018) (end 152.428982 42.218832) (width 1) (layer "F.Cu") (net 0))
 (segment (start 148.852162 30.287838) (end 149.948 29.192) (width 1) (layer "F.Cu") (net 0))
 (segment (start 142.750047 3.556) (end 158.712908 19.518861) (width 1) (layer "F.Cu") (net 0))
 (segment (start 23.622 19.056) (end 27.178 22.612) (width 6) (layer "F.Cu") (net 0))
 (segment (start 60.477525 11.306) (end 56.122 11.306) (width 4.13) (layer "F.Cu") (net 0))
 (segment (start 146.196058 15.093942) (end 143.303582 15.093942) (width 1) (layer "F.Cu") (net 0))
 (segment (start 149.948 24.992) (end 147.669942 22.713942) (width 1) (layer "F.Cu") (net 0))
 (segment (start 127.762 57.912) (end 134.516 57.912) (width 6) (layer "F.Cu") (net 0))
 (segment (start 140.895687 53.752127) (end 64.767397 53.752127) (width 1) (layer "F.Cu") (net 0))
 (segment (start 127.762 3.81) (end 134.368 3.81) (width 6) (layer "F.Cu") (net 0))
 (segment (start 64.767397 53.752127) (end 64.563582 53.955942) (width 1) (layer "F.Cu") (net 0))
 (segment (start 154.864137 20.792) (end 141.54608 7.473942) (width 1) (layer "F.Cu") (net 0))
 (segment (start 139.967721 57.729125) (end 134.698875 57.729125) (width 1) (layer "F.Cu") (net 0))
 (segment (start 56.122 3.556) (end 56.122 11.306) (width 4.13) (layer "F.Cu") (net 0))
 (segment (start 147.669942 22.713942) (end 105.779942 22.713942) (width 1) (layer "F.Cu") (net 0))
 (segment (start 134.698875 57.729125) (end 134.622 57.806) (width 1) (layer "F.Cu") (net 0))
 (segment (start 20.32 6.858) (end 23.622 3.556) (width 6) (layer "F.Cu") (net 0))
 (segment (start 149.948 33.392) (end 144.965599 38.374401) (width 1) (layer "F.Cu") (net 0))
 (segment (start 158.712908 22.83521) (end 156.556118 24.992) (width 1) (layer "F.Cu") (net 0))
 (segment (start 155.448 42.248846) (end 139.967721 57.729125) (width 1) (layer "F.Cu") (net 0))
 (segment (start 102.122 57.806) (end 109.114 57.806) (width 6) (layer "F.Cu") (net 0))
 (segment (start 134.622 3.556) (end 142.750047 3.556) (width 1) (layer "F.Cu") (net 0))
 (segment (start 149.948 19.057461) (end 146.09027 15.19973) (width 1) (layer "F.Cu") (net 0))
 (segment (start 106.053599 38.374401) (end 105.966058 38.461942) (width 1) (layer "F.Cu") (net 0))
 (segment (start 155.448 37.592) (end 155.448 42.248846) (width 1) (layer "F.Cu") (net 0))
 (segment (start 158.712908 19.518861) (end 158.712908 22.83521) (width 1) (layer "F.Cu") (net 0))
 (segment (start 20.32 22.358) (end 23.622 19.056) (width 6) (layer "F.Cu") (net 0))
 (segment (start 56.122 3.556) (end 60.39164 3.556) (width 4.13) (layer "F.Cu") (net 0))
 (segment (start 155.448 33.392) (end 152.428982 36.411018) (width 1) (layer "F.Cu") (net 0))
 (segment (start 149.910216 37.629784) (end 149.910216 41.821133) (width 1) (layer "F.Cu") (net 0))
 (segment (start 149.910216 41.821133) (end 145.649407 46.081942) (width 1) (layer "F.Cu") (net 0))
 (segment (start 64.309582 7.473942) (end 60.477525 11.306) (width 4.13) (layer "F.Cu") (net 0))
 (segment (start 134.368 3.81) (end 134.622 3.556) (width 6) (layer "F.Cu") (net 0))
 (segment (start 144.965599 38.374401) (end 106.053599 38.374401) (width 1) (layer "F.Cu") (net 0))
 (segment (start 60.39164 3.556) (end 64.309582 7.473942) (width 4.13) (layer "F.Cu") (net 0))
 (segment (start 149.948 20.792) (end 149.948 19.057461) (width 1) (layer "F.Cu") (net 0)))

